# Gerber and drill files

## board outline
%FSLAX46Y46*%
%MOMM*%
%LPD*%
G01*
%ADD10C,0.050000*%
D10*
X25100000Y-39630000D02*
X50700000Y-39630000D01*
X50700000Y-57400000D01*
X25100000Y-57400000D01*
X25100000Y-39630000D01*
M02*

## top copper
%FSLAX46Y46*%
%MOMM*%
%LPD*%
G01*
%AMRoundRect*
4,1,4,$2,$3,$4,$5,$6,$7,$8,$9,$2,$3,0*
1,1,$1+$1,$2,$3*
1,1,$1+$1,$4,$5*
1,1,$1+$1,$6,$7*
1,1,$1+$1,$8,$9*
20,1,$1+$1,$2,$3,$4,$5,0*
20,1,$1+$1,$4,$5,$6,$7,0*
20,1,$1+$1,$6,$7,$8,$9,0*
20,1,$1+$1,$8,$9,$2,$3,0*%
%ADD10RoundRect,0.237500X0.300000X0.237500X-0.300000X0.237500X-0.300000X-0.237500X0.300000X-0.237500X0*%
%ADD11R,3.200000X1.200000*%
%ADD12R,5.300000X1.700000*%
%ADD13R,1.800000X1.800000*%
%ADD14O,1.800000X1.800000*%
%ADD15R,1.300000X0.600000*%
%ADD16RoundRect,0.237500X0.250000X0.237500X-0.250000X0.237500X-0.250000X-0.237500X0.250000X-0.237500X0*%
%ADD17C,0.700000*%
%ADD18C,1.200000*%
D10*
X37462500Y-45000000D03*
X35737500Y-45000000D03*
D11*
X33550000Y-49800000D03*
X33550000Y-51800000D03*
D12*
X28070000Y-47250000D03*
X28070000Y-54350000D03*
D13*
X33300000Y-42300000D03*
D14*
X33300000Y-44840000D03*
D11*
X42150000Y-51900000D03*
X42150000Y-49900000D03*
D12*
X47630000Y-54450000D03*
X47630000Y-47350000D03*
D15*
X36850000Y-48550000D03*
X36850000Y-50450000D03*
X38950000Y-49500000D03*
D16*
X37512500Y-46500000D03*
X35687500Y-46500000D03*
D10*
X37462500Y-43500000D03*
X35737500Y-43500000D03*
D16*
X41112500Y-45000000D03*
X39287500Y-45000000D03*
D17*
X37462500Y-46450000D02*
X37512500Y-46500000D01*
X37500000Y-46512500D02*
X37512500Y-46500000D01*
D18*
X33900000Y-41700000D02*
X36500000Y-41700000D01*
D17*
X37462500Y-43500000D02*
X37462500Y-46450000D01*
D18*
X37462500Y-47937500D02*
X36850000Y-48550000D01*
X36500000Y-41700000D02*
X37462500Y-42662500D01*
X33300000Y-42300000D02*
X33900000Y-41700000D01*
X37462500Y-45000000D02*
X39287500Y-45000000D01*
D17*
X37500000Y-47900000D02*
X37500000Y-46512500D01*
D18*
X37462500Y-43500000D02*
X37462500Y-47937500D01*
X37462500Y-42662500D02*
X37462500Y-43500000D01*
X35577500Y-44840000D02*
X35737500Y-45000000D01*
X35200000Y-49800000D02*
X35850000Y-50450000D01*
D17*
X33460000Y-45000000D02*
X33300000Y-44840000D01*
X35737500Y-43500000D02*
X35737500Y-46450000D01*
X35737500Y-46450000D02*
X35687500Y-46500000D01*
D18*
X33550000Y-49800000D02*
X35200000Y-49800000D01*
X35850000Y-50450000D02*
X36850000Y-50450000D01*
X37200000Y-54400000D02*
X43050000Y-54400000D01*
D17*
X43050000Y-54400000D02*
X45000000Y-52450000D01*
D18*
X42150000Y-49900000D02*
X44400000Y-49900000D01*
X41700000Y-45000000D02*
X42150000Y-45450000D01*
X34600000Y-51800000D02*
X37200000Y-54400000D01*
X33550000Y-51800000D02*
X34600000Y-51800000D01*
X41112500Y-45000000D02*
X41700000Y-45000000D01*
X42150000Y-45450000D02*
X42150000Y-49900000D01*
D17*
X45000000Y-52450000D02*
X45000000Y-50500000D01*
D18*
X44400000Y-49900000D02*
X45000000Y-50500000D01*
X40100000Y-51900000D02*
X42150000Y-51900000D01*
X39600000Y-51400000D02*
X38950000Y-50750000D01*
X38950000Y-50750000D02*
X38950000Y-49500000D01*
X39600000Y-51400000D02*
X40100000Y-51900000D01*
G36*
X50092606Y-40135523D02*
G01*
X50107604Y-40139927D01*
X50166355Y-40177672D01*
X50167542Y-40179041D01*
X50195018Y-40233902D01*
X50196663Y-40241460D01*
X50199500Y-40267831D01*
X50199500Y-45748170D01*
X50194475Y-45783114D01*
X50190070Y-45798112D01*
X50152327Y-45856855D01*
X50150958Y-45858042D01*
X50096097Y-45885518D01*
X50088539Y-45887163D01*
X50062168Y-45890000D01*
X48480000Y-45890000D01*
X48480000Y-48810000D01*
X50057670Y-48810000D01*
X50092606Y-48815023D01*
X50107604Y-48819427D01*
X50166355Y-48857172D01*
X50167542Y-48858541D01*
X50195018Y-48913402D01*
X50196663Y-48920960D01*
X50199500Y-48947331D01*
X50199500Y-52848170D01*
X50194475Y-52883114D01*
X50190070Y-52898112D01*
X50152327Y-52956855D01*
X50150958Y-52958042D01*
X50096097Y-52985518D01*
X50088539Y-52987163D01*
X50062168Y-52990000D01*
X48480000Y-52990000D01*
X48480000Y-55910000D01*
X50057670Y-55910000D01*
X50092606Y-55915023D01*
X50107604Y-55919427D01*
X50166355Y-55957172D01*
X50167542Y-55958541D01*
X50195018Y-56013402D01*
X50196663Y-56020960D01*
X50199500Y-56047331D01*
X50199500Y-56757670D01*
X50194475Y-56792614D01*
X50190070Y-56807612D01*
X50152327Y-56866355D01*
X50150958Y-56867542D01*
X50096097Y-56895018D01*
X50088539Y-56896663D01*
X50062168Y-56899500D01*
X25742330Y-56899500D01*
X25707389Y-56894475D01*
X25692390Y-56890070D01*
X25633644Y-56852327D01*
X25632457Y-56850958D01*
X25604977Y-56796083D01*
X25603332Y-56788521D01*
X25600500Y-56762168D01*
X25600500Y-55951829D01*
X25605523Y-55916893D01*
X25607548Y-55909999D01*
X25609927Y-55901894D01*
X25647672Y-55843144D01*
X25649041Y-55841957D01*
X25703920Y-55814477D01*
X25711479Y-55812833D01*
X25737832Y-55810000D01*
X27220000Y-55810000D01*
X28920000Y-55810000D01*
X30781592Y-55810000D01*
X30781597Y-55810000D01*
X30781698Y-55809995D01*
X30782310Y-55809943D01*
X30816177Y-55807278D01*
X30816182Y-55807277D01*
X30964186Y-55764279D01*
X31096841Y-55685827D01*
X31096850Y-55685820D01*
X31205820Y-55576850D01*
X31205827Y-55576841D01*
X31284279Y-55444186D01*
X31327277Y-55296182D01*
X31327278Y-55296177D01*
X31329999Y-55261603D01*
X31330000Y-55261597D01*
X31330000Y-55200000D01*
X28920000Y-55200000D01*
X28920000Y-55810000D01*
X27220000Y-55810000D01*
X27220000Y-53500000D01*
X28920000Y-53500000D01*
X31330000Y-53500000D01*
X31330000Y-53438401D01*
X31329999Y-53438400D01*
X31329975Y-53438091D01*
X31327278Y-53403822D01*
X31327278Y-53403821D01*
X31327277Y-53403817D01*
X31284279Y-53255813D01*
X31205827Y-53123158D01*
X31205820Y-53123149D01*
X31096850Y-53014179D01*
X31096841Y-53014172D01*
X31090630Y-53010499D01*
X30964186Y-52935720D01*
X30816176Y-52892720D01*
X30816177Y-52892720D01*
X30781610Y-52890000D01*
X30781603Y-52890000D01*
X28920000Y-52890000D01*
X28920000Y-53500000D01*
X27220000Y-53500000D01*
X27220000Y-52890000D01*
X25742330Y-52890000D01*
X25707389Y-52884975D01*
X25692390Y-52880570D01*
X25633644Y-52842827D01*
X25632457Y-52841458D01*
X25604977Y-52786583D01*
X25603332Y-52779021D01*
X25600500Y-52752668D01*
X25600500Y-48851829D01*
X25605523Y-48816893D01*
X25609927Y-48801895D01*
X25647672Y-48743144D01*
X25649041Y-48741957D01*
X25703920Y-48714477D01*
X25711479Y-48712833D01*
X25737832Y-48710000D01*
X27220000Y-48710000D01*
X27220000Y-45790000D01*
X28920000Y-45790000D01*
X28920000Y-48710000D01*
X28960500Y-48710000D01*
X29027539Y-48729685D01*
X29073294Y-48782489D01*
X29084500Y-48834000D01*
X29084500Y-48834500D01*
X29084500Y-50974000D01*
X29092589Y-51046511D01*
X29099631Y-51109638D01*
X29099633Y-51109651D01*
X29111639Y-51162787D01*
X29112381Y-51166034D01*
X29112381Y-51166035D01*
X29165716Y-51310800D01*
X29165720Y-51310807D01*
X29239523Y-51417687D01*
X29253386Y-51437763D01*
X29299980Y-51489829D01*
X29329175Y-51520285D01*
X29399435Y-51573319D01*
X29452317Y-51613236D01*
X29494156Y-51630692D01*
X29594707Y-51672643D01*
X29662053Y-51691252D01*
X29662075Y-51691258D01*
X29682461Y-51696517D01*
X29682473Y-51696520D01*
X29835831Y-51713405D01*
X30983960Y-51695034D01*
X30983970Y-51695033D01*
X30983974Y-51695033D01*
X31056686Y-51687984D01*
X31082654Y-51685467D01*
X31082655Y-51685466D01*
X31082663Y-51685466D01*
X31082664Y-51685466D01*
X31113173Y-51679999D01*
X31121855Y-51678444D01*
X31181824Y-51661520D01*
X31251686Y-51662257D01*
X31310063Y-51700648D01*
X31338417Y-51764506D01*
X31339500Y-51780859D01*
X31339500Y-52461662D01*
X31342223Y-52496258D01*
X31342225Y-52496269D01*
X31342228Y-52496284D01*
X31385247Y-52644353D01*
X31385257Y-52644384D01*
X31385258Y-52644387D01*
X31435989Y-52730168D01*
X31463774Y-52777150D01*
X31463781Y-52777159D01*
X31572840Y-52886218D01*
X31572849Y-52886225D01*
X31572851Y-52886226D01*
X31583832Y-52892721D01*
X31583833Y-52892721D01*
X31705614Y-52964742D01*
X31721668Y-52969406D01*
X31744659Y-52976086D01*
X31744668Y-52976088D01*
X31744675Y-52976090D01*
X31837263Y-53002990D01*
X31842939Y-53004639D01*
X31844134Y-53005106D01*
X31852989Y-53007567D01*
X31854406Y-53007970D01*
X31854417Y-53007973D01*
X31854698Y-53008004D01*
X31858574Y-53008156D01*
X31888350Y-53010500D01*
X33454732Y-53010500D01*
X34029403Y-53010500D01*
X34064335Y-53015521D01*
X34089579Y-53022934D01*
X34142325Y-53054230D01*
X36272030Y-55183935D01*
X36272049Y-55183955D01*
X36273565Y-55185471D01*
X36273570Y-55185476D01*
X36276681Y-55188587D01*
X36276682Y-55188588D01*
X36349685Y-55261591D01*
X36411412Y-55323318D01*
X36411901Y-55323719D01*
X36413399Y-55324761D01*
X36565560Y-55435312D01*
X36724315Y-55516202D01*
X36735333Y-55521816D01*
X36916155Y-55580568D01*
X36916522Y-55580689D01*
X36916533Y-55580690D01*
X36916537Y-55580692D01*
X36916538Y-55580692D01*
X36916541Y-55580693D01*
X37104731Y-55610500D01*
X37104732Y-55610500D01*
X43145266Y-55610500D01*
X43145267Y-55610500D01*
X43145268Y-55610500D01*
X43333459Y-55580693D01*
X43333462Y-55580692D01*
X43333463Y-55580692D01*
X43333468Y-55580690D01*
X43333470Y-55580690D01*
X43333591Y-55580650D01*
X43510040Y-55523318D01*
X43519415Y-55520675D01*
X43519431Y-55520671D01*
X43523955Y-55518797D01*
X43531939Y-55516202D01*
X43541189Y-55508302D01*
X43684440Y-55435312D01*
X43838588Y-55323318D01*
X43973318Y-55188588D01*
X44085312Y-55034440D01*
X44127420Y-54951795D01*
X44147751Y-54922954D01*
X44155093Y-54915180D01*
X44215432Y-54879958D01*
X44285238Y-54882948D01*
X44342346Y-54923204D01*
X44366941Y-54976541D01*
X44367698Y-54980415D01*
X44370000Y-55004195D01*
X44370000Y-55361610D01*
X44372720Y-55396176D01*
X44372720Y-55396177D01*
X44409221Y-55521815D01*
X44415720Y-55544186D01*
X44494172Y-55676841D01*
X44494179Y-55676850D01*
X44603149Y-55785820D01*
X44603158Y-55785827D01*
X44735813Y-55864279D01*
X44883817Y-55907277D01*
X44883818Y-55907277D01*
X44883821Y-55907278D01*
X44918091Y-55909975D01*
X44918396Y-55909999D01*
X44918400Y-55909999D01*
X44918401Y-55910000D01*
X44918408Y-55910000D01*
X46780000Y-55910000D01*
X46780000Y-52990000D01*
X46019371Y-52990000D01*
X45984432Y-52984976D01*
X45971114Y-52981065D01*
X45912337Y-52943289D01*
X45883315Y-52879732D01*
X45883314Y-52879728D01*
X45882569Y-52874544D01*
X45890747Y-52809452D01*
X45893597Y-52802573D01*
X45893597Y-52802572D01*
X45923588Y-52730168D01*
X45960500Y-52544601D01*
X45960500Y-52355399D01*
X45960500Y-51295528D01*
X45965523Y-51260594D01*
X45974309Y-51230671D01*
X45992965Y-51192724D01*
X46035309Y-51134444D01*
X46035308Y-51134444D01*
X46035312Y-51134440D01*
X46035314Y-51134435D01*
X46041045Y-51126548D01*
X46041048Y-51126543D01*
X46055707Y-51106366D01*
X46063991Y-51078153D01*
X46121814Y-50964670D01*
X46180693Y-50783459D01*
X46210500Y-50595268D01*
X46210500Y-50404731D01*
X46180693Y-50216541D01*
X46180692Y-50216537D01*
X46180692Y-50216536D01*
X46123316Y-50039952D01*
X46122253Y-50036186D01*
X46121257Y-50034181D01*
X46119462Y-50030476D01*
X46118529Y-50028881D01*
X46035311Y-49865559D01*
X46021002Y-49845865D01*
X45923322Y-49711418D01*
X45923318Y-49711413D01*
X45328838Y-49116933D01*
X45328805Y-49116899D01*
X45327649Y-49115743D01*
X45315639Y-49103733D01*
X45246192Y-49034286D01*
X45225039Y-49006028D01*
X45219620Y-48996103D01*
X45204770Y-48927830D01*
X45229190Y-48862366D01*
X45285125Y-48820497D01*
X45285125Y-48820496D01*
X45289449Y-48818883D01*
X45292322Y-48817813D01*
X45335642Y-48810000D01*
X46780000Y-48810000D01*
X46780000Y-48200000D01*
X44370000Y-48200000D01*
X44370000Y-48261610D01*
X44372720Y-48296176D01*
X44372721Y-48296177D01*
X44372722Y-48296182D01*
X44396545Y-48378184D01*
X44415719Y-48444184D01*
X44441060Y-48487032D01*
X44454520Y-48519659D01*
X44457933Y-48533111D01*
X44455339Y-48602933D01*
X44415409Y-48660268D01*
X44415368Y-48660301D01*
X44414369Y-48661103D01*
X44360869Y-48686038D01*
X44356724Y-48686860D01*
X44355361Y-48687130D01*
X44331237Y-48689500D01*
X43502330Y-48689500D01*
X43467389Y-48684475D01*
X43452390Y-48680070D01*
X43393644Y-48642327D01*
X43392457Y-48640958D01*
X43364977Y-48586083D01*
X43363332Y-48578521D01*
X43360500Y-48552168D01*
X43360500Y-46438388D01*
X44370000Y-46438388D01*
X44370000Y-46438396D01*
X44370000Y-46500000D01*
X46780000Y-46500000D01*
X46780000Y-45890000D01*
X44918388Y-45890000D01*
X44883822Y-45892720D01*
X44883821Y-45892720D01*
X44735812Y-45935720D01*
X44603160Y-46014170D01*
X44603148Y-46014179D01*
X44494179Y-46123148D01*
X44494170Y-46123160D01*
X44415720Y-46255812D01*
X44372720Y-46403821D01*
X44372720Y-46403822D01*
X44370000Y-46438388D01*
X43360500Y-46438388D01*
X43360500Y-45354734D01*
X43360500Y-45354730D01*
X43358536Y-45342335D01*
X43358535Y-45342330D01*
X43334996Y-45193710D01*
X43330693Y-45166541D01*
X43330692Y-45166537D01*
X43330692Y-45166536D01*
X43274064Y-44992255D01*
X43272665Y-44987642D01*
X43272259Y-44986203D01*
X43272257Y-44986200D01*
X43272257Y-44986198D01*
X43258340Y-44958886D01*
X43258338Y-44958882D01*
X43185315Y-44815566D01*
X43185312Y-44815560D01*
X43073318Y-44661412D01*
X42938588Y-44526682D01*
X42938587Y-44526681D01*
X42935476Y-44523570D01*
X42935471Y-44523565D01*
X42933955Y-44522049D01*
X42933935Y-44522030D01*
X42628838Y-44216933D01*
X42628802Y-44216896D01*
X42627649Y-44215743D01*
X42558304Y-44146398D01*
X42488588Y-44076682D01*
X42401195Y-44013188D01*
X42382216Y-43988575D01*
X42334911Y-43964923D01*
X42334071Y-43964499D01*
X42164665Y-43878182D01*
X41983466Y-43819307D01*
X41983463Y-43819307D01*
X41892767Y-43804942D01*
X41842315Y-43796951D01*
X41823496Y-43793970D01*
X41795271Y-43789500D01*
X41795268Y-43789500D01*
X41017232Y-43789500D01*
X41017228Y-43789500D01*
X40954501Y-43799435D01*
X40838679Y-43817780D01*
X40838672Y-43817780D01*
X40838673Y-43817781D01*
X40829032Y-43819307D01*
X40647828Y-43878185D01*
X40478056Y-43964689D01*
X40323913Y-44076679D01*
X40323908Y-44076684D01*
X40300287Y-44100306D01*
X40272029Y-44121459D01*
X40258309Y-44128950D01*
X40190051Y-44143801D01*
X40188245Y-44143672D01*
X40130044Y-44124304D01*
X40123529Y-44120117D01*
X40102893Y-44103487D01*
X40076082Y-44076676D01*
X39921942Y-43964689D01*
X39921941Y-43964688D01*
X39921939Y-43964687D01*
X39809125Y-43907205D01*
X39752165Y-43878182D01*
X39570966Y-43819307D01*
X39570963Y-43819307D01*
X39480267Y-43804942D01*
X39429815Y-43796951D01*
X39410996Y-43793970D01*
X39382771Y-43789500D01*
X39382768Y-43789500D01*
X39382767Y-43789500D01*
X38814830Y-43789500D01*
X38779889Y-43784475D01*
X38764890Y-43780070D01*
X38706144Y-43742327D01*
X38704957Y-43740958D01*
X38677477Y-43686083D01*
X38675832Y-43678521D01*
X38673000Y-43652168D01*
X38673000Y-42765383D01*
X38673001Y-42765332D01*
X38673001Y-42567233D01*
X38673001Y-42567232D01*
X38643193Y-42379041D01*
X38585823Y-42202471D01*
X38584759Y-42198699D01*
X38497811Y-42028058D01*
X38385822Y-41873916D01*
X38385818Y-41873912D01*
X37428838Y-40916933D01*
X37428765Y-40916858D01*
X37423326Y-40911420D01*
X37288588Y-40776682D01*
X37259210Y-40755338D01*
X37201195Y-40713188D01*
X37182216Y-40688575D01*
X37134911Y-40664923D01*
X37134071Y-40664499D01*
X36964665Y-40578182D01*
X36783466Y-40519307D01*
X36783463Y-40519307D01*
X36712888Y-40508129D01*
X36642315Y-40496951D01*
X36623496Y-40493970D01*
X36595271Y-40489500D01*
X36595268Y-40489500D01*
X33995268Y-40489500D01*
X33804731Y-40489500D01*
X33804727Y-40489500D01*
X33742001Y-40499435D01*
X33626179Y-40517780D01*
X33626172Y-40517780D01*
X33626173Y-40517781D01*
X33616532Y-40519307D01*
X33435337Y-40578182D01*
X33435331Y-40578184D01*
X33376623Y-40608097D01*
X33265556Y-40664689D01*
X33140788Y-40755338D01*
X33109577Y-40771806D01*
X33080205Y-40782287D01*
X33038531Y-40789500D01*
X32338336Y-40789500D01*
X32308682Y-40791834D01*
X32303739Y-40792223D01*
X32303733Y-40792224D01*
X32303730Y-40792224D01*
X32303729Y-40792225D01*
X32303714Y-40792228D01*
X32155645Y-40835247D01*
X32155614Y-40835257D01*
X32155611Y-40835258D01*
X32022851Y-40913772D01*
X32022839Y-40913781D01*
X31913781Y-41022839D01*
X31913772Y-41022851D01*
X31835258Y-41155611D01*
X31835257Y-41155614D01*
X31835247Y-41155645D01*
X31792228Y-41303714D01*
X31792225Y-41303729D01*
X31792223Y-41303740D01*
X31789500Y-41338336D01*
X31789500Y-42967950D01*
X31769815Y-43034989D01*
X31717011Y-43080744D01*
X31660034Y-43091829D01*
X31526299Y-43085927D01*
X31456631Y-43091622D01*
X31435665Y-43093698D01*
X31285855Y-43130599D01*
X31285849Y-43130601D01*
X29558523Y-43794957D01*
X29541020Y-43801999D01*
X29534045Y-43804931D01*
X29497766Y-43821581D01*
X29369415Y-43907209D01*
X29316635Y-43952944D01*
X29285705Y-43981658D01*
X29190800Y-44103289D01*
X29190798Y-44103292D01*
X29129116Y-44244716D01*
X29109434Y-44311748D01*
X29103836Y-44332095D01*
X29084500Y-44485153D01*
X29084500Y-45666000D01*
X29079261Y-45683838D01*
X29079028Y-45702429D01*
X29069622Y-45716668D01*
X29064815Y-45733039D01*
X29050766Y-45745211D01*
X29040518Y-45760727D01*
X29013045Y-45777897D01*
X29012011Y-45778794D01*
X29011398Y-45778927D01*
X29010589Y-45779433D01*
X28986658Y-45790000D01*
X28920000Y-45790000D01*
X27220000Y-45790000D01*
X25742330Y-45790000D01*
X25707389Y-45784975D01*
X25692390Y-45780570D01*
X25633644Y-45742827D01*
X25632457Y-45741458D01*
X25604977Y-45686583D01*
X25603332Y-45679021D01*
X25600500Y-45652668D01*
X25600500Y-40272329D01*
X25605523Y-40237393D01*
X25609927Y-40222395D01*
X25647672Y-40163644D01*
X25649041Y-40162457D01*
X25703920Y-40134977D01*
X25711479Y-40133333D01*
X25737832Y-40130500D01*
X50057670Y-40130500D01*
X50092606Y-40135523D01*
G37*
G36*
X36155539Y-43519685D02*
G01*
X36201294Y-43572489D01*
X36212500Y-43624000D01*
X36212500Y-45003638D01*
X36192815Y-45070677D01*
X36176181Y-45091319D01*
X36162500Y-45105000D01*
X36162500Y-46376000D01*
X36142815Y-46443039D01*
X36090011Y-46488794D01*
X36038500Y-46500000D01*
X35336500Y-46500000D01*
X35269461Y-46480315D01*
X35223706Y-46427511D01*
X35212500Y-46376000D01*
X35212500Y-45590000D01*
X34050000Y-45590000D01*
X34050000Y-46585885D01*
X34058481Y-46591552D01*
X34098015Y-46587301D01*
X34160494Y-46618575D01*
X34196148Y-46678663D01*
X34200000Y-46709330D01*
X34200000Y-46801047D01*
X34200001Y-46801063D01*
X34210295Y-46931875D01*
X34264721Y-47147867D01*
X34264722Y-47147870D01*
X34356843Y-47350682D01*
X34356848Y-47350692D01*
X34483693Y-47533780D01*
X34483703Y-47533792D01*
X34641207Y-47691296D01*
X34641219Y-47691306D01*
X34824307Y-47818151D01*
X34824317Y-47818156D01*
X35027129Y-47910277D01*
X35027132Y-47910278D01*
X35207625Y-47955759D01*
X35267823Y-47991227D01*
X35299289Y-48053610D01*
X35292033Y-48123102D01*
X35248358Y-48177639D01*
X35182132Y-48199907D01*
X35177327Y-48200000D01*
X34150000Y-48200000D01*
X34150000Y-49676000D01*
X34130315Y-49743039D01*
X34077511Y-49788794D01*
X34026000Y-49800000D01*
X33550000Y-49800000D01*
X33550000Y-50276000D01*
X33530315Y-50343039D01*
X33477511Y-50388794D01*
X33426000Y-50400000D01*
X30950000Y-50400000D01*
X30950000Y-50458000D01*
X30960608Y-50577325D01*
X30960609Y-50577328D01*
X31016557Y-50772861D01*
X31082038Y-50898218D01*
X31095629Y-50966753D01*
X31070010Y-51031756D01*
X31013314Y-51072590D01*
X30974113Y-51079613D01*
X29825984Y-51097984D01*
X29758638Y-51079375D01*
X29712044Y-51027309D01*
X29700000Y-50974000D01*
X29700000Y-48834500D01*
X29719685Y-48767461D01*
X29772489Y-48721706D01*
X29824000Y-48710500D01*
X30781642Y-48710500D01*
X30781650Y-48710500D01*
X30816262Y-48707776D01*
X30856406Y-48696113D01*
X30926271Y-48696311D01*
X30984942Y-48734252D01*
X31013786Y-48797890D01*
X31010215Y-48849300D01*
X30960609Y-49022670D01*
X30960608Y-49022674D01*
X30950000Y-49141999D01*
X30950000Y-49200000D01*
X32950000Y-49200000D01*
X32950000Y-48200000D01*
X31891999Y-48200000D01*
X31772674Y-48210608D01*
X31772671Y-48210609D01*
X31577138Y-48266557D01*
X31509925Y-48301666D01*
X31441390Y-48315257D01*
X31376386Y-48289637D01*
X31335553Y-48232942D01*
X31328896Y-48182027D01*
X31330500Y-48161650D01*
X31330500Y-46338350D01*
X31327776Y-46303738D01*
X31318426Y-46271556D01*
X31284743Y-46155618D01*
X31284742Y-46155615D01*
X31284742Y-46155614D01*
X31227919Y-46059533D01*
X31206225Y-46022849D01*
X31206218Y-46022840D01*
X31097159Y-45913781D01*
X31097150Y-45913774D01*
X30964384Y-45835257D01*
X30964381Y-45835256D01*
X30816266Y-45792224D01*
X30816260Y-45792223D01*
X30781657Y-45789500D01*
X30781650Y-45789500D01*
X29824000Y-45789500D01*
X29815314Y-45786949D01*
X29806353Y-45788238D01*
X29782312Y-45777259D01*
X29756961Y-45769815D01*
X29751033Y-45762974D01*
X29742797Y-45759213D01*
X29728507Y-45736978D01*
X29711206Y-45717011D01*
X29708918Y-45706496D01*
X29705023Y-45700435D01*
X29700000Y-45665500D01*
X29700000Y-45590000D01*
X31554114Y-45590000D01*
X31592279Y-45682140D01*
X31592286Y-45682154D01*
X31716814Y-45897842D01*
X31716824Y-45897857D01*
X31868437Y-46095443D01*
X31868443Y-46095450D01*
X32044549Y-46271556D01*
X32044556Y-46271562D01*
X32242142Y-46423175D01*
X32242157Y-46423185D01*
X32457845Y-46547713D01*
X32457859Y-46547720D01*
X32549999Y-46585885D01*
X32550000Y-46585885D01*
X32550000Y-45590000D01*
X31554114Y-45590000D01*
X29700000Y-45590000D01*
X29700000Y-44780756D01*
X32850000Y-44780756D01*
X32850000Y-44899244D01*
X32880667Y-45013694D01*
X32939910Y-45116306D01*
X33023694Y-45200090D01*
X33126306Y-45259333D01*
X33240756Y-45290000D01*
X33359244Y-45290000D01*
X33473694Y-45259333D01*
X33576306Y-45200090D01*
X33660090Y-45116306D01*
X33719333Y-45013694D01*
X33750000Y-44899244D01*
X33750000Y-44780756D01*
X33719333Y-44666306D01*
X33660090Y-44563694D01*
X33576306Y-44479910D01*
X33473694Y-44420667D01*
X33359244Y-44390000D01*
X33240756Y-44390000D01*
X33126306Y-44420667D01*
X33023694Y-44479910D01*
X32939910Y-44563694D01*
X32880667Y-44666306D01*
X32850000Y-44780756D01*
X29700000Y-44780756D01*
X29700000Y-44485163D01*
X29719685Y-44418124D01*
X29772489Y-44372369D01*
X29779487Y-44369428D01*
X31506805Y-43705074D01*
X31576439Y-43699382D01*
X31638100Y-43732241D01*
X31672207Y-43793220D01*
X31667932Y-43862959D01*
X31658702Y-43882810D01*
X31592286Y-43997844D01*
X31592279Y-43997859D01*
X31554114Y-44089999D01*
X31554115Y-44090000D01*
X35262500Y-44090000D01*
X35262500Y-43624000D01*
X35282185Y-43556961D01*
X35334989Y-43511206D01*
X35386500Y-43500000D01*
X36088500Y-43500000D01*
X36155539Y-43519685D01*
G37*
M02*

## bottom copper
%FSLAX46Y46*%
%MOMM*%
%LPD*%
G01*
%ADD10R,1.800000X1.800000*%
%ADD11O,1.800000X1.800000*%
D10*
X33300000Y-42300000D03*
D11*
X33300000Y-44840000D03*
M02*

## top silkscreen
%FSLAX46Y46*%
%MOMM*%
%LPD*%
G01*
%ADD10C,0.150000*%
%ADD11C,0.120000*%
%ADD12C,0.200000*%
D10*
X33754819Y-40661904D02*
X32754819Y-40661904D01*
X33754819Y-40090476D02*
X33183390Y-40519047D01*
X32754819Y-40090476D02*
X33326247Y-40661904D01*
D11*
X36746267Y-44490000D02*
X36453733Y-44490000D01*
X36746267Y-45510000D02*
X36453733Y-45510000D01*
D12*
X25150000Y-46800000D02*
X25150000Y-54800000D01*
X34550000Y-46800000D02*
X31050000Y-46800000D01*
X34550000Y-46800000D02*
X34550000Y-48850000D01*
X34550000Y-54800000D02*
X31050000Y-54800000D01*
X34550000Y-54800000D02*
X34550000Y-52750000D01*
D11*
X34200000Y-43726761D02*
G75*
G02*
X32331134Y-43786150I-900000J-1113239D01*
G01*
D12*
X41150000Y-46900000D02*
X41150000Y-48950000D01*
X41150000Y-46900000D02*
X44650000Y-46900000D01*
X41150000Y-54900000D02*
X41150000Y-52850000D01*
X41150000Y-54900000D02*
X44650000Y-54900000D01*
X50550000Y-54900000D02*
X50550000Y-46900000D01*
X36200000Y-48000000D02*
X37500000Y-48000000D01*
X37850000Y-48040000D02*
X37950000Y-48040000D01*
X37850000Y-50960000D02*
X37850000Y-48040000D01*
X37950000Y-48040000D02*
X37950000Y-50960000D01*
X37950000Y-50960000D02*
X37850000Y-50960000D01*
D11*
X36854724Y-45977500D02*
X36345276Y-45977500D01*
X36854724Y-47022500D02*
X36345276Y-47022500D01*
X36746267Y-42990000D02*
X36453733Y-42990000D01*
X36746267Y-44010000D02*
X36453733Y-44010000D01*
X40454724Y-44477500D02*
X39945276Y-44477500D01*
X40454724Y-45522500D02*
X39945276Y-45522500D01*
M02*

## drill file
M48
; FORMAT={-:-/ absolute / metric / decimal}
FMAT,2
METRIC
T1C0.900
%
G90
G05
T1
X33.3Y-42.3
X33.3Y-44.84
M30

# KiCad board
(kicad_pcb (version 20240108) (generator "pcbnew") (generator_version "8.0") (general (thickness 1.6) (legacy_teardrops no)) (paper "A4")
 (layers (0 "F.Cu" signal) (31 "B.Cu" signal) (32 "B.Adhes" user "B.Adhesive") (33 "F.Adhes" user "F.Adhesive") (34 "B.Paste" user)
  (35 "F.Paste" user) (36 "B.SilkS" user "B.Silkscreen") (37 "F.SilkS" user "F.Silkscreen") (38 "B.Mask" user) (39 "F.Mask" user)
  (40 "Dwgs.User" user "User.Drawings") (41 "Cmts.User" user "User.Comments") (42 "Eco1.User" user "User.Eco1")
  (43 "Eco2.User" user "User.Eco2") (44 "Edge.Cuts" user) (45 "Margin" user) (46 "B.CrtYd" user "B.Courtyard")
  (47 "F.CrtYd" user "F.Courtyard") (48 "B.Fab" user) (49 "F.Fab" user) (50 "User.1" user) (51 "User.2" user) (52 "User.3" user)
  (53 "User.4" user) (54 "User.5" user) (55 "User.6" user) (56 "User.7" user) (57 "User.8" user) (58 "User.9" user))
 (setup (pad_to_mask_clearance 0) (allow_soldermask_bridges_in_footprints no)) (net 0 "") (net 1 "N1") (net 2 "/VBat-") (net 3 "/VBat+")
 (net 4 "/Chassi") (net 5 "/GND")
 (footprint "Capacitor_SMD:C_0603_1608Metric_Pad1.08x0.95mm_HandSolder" (layer "F.Cu") (at 36.6 45 180)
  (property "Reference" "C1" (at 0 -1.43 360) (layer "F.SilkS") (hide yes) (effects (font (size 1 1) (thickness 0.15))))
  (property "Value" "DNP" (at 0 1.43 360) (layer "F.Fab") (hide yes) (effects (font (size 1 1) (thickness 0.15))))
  (fp_line (start -0.146267 0.51) (end 0.146267 0.51) (stroke (width 0.12) (type solid)) (layer "F.SilkS"))
  (fp_line (start -0.146267 -0.51) (end 0.146267 -0.51) (stroke (width 0.12) (type solid)) (layer "F.SilkS"))
  (pad "1" smd roundrect (at -0.8625 0 180) (size 1.075 0.95) (layers "F.Cu" "F.Paste" "F.Mask") (roundrect_rratio 0.25) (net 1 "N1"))
  (pad "2" smd roundrect (at 0.8625 0 180) (size 1.075 0.95) (layers "F.Cu" "F.Paste" "F.Mask") (roundrect_rratio 0.25) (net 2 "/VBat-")))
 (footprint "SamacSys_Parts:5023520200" (layer "F.Cu") (at 34.55 50.8 -90)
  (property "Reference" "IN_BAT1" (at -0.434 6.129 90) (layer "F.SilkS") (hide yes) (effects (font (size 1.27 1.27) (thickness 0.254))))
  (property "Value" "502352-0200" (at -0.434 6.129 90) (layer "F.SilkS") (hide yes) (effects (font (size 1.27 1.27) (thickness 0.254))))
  (fp_line (start -4 9.4) (end 4 9.4) (stroke (width 0.2) (type solid)) (layer "F.SilkS"))
  (fp_line (start -4 0) (end -4 3.5) (stroke (width 0.2) (type solid)) (layer "F.SilkS"))
  (fp_line (start -4 0) (end -1.95 0) (stroke (width 0.2) (type solid)) (layer "F.SilkS"))
  (fp_line (start 4 0) (end 4 3.5) (stroke (width 0.2) (type solid)) (layer "F.SilkS"))
  (fp_line (start 4 0) (end 1.95 0) (stroke (width 0.2) (type solid)) (layer "F.SilkS"))
  (pad "1" smd rect (at -1 1 270) (size 1.2 3.2) (layers "F.Cu" "F.Paste" "F.Mask") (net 2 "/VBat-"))
  (pad "2" smd rect (at 1 1 270) (size 1.2 3.2) (layers "F.Cu" "F.Paste" "F.Mask") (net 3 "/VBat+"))
  (pad "3" smd rect (at -3.55 6.48 270) (size 1.7 5.3) (layers "F.Cu" "F.Paste" "F.Mask") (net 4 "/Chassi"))
  (pad "4" smd rect (at 3.55 6.48 270) (size 1.7 5.3) (layers "F.Cu" "F.Paste" "F.Mask") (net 4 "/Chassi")))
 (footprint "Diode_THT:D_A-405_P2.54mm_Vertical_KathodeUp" (layer "F.Cu") (at 33.3 42.3 -90)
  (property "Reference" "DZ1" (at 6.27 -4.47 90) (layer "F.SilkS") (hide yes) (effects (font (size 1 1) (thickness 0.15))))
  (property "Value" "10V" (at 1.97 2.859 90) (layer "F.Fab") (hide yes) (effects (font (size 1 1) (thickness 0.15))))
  (fp_arc (start 1.426761 -0.9) (mid 3.970816 -0.045469) (end 1.48615 0.968866) (stroke (width 0.12) (type solid)) (layer "F.SilkS"))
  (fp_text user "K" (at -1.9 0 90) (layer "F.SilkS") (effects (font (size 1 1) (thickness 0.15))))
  (pad "1" thru_hole rect (at 0 0 270) (size 1.8 1.8) (drill 0.9) (layers "*.Cu" "*.Mask") (remove_unused_layers no) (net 1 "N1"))
  (pad "2" thru_hole oval (at 2.54 0 270) (size 1.8 1.8) (drill 0.9) (layers "*.Cu" "*.Mask") (remove_unused_layers no) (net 2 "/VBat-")))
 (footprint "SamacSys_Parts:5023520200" (layer "F.Cu") (at 41.15 50.9 90)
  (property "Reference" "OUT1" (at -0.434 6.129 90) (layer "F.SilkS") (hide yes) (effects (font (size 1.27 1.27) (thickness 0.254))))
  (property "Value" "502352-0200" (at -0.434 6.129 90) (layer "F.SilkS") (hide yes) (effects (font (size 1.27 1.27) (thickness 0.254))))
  (fp_line (start 4 0) (end 1.95 0) (stroke (width 0.2) (type solid)) (layer "F.SilkS"))
  (fp_line (start 4 0) (end 4 3.5) (stroke (width 0.2) (type solid)) (layer "F.SilkS"))
  (fp_line (start -4 0) (end -1.95 0) (stroke (width 0.2) (type solid)) (layer "F.SilkS"))
  (fp_line (start -4 0) (end -4 3.5) (stroke (width 0.2) (type solid)) (layer "F.SilkS"))
  (fp_line (start -4 9.4) (end 4 9.4) (stroke (width 0.2) (type solid)) (layer "F.SilkS"))
  (pad "1" smd rect (at -1 1 90) (size 1.2 3.2) (layers "F.Cu" "F.Paste" "F.Mask") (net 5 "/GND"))
  (pad "2" smd rect (at 1 1 90) (size 1.2 3.2) (layers "F.Cu" "F.Paste" "F.Mask") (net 3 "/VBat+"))
  (pad "3" smd rect (at -3.55 6.48 90) (size 1.7 5.3) (layers "F.Cu" "F.Paste" "F.Mask") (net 4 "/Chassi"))
  (pad "4" smd rect (at 3.55 6.48 90) (size 1.7 5.3) (layers "F.Cu" "F.Paste" "F.Mask") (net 4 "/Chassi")))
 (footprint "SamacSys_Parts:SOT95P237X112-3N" (layer "F.Cu") (at 37.9 49.5)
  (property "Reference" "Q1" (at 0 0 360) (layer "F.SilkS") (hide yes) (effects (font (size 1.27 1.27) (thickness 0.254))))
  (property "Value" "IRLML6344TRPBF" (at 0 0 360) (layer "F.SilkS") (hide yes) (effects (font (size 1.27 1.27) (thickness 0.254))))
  (fp_line (start -1.7 -1.5) (end -0.4 -1.5) (stroke (width 0.2) (type solid)) (layer "F.SilkS"))
  (fp_line (start -0.05 -1.46) (end 0.05 -1.46) (stroke (width 0.2) (type solid)) (layer "F.SilkS"))
  (fp_line (start -0.05 1.46) (end -0.05 -1.46) (stroke (width 0.2) (type solid)) (layer "F.SilkS"))
  (fp_line (start 0.05 -1.46) (end 0.05 1.46) (stroke (width 0.2) (type solid)) (layer "F.SilkS"))
  (fp_line (start 0.05 1.46) (end -0.05 1.46) (stroke (width 0.2) (type solid)) (layer "F.SilkS"))
  (pad "1" smd rect (at -1.05 -0.95 90) (size 0.6 1.3) (layers "F.Cu" "F.Paste" "F.Mask") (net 1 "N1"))
  (pad "2" smd rect (at -1.05 0.95 90) (size 0.6 1.3) (layers "F.Cu" "F.Paste" "F.Mask") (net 2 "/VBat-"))
  (pad "3" smd rect (at 1.05 0 90) (size 0.6 1.3) (layers "F.Cu" "F.Paste" "F.Mask") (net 5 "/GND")))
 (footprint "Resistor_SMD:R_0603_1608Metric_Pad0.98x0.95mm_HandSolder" (layer "F.Cu") (at 36.6 46.5 180)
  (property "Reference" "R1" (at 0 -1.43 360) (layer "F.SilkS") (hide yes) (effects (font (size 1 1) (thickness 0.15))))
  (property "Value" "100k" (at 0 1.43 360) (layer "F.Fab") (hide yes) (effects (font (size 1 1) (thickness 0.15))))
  (fp_line (start -0.254724 0.5225) (end 0.254724 0.5225) (stroke (width 0.12) (type solid)) (layer "F.SilkS"))
  (fp_line (start -0.254724 -0.5225) (end 0.254724 -0.5225) (stroke (width 0.12) (type solid)) (layer "F.SilkS"))
  (pad "1" smd roundrect (at -0.9125 0 180) (size 0.975 0.95) (layers "F.Cu" "F.Paste" "F.Mask") (roundrect_rratio 0.25) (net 1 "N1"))
  (pad "2" smd roundrect (at 0.9125 0 180) (size 0.975 0.95) (layers "F.Cu" "F.Paste" "F.Mask") (roundrect_rratio 0.25) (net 2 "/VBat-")))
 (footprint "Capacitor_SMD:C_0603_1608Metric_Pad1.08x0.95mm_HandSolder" (layer "F.Cu") (at 36.6 43.5 180)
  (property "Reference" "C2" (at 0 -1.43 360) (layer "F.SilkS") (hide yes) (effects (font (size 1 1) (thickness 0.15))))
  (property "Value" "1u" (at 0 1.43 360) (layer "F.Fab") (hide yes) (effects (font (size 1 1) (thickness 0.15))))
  (fp_line (start -0.146267 0.51) (end 0.146267 0.51) (stroke (width 0.12) (type solid)) (layer "F.SilkS"))
  (fp_line (start -0.146267 -0.51) (end 0.146267 -0.51) (stroke (width 0.12) (type solid)) (layer "F.SilkS"))
  (pad "1" smd roundrect (at -0.8625 0 180) (size 1.075 0.95) (layers "F.Cu" "F.Paste" "F.Mask") (roundrect_rratio 0.25) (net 1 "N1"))
  (pad "2" smd roundrect (at 0.8625 0 180) (size 1.075 0.95) (layers "F.Cu" "F.Paste" "F.Mask") (roundrect_rratio 0.25) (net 2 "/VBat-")))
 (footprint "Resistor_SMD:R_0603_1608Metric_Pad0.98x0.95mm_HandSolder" (layer "F.Cu") (at 40.2 45 180)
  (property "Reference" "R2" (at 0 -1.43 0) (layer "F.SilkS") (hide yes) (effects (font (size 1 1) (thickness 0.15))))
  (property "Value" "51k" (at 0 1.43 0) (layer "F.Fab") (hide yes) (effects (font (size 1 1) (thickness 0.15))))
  (fp_line (start -0.254724 0.5225) (end 0.254724 0.5225) (stroke (width 0.12) (type solid)) (layer "F.SilkS"))
  (fp_line (start -0.254724 -0.5225) (end 0.254724 -0.5225) (stroke (width 0.12) (type solid)) (layer "F.SilkS"))
  (pad "1" smd roundrect (at -0.9125 0 180) (size 0.975 0.95) (layers "F.Cu" "F.Paste" "F.Mask") (roundrect_rratio 0.25) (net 3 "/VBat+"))
  (pad "2" smd roundrect (at 0.9125 0 180) (size 0.975 0.95) (layers "F.Cu" "F.Paste" "F.Mask") (roundrect_rratio 0.25) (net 1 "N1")))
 (gr_rect (start 25.1 39.63) (end 50.7 57.4) (stroke (width 0.05) (type default)) (fill none) (layer "Edge.Cuts"))
 (segment (start 37.4625 46.45) (end 37.5125 46.5) (width 0.7) (layer "F.Cu") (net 1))
 (segment (start 37.5 46.5125) (end 37.5125 46.5) (width 0.7) (layer "F.Cu") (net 1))
 (segment (start 33.9 41.7) (end 36.5 41.7) (width 1.2) (layer "F.Cu") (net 1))
 (segment (start 37.4625 43.5) (end 37.4625 46.45) (width 0.7) (layer "F.Cu") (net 1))
 (segment (start 37.4625 47.9375) (end 36.85 48.55) (width 1.2) (layer "F.Cu") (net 1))
 (segment (start 36.5 41.7) (end 37.4625 42.6625) (width 1.2) (layer "F.Cu") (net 1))
 (segment (start 33.3 42.3) (end 33.9 41.7) (width 1.2) (layer "F.Cu") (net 1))
 (segment (start 37.4625 45) (end 39.2875 45) (width 1.2) (layer "F.Cu") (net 1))
 (segment (start 37.5 47.9) (end 37.5 46.5125) (width 0.7) (layer "F.Cu") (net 1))
 (segment (start 37.4625 43.5) (end 37.4625 47.9375) (width 1.2) (layer "F.Cu") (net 1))
 (segment (start 37.4625 42.6625) (end 37.4625 43.5) (width 1.2) (layer "F.Cu") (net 1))
 (segment (start 35.5775 44.84) (end 35.7375 45) (width 1.2) (layer "F.Cu") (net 2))
 (segment (start 35.2 49.8) (end 35.85 50.45) (width 1.2) (layer "F.Cu") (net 2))
 (segment (start 33.46 45) (end 33.3 44.84) (width 0.7) (layer "F.Cu") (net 2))
 (segment (start 35.7375 43.5) (end 35.7375 46.45) (width 0.7) (layer "F.Cu") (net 2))
 (segment (start 35.7375 46.45) (end 35.6875 46.5) (width 0.7) (layer "F.Cu") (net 2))
 (segment (start 33.55 49.8) (end 35.2 49.8) (width 1.2) (layer "F.Cu") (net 2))
 (segment (start 35.85 50.45) (end 36.85 50.45) (width 1.2) (layer "F.Cu") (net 2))
 (segment (start 37.2 54.4) (end 43.05 54.4) (width 1.2) (layer "F.Cu") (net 3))
 (segment (start 43.05 54.4) (end 45 52.45) (width 0.7) (layer "F.Cu") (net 3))
 (segment (start 42.15 49.9) (end 44.4 49.9) (width 1.2) (layer "F.Cu") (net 3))
 (segment (start 41.7 45) (end 42.15 45.45) (width 1.2) (layer "F.Cu") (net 3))
 (segment (start 34.6 51.8) (end 37.2 54.4) (width 1.2) (layer "F.Cu") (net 3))
 (segment (start 33.55 51.8) (end 34.6 51.8) (width 1.2) (layer "F.Cu") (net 3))
 (segment (start 41.1125 45) (end 41.7 45) (width 1.2) (layer "F.Cu") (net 3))
 (segment (start 42.15 45.45) (end 42.15 49.9) (width 1.2) (layer "F.Cu") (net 3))
 (segment (start 45 52.45) (end 45 50.5) (width 0.7) (layer "F.Cu") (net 3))
 (segment (start 44.4 49.9) (end 45 50.5) (width 1.2) (layer "F.Cu") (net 3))
 (segment (start 40.1 51.9) (end 42.15 51.9) (width 1.2) (layer "F.Cu") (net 5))
 (segment (start 39.6 51.4) (end 38.95 50.75) (width 1.2) (layer "F.Cu") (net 5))
 (segment (start 38.95 50.75) (end 38.95 49.5) (width 1.2) (layer "F.Cu") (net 5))
 (segment (start 39.6 51.4) (end 40.1 51.9) (width 1.2) (layer "F.Cu") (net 5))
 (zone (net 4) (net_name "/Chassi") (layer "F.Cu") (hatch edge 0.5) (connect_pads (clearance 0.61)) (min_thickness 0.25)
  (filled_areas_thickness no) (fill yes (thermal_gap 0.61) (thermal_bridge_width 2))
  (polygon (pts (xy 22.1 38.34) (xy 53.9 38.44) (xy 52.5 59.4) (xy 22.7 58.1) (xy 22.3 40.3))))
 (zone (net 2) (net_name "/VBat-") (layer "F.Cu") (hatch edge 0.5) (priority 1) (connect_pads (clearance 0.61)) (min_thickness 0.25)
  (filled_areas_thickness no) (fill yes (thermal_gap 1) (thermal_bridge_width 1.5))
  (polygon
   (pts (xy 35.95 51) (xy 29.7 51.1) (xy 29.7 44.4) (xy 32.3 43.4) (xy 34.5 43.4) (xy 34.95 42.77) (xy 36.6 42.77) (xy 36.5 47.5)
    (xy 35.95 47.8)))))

